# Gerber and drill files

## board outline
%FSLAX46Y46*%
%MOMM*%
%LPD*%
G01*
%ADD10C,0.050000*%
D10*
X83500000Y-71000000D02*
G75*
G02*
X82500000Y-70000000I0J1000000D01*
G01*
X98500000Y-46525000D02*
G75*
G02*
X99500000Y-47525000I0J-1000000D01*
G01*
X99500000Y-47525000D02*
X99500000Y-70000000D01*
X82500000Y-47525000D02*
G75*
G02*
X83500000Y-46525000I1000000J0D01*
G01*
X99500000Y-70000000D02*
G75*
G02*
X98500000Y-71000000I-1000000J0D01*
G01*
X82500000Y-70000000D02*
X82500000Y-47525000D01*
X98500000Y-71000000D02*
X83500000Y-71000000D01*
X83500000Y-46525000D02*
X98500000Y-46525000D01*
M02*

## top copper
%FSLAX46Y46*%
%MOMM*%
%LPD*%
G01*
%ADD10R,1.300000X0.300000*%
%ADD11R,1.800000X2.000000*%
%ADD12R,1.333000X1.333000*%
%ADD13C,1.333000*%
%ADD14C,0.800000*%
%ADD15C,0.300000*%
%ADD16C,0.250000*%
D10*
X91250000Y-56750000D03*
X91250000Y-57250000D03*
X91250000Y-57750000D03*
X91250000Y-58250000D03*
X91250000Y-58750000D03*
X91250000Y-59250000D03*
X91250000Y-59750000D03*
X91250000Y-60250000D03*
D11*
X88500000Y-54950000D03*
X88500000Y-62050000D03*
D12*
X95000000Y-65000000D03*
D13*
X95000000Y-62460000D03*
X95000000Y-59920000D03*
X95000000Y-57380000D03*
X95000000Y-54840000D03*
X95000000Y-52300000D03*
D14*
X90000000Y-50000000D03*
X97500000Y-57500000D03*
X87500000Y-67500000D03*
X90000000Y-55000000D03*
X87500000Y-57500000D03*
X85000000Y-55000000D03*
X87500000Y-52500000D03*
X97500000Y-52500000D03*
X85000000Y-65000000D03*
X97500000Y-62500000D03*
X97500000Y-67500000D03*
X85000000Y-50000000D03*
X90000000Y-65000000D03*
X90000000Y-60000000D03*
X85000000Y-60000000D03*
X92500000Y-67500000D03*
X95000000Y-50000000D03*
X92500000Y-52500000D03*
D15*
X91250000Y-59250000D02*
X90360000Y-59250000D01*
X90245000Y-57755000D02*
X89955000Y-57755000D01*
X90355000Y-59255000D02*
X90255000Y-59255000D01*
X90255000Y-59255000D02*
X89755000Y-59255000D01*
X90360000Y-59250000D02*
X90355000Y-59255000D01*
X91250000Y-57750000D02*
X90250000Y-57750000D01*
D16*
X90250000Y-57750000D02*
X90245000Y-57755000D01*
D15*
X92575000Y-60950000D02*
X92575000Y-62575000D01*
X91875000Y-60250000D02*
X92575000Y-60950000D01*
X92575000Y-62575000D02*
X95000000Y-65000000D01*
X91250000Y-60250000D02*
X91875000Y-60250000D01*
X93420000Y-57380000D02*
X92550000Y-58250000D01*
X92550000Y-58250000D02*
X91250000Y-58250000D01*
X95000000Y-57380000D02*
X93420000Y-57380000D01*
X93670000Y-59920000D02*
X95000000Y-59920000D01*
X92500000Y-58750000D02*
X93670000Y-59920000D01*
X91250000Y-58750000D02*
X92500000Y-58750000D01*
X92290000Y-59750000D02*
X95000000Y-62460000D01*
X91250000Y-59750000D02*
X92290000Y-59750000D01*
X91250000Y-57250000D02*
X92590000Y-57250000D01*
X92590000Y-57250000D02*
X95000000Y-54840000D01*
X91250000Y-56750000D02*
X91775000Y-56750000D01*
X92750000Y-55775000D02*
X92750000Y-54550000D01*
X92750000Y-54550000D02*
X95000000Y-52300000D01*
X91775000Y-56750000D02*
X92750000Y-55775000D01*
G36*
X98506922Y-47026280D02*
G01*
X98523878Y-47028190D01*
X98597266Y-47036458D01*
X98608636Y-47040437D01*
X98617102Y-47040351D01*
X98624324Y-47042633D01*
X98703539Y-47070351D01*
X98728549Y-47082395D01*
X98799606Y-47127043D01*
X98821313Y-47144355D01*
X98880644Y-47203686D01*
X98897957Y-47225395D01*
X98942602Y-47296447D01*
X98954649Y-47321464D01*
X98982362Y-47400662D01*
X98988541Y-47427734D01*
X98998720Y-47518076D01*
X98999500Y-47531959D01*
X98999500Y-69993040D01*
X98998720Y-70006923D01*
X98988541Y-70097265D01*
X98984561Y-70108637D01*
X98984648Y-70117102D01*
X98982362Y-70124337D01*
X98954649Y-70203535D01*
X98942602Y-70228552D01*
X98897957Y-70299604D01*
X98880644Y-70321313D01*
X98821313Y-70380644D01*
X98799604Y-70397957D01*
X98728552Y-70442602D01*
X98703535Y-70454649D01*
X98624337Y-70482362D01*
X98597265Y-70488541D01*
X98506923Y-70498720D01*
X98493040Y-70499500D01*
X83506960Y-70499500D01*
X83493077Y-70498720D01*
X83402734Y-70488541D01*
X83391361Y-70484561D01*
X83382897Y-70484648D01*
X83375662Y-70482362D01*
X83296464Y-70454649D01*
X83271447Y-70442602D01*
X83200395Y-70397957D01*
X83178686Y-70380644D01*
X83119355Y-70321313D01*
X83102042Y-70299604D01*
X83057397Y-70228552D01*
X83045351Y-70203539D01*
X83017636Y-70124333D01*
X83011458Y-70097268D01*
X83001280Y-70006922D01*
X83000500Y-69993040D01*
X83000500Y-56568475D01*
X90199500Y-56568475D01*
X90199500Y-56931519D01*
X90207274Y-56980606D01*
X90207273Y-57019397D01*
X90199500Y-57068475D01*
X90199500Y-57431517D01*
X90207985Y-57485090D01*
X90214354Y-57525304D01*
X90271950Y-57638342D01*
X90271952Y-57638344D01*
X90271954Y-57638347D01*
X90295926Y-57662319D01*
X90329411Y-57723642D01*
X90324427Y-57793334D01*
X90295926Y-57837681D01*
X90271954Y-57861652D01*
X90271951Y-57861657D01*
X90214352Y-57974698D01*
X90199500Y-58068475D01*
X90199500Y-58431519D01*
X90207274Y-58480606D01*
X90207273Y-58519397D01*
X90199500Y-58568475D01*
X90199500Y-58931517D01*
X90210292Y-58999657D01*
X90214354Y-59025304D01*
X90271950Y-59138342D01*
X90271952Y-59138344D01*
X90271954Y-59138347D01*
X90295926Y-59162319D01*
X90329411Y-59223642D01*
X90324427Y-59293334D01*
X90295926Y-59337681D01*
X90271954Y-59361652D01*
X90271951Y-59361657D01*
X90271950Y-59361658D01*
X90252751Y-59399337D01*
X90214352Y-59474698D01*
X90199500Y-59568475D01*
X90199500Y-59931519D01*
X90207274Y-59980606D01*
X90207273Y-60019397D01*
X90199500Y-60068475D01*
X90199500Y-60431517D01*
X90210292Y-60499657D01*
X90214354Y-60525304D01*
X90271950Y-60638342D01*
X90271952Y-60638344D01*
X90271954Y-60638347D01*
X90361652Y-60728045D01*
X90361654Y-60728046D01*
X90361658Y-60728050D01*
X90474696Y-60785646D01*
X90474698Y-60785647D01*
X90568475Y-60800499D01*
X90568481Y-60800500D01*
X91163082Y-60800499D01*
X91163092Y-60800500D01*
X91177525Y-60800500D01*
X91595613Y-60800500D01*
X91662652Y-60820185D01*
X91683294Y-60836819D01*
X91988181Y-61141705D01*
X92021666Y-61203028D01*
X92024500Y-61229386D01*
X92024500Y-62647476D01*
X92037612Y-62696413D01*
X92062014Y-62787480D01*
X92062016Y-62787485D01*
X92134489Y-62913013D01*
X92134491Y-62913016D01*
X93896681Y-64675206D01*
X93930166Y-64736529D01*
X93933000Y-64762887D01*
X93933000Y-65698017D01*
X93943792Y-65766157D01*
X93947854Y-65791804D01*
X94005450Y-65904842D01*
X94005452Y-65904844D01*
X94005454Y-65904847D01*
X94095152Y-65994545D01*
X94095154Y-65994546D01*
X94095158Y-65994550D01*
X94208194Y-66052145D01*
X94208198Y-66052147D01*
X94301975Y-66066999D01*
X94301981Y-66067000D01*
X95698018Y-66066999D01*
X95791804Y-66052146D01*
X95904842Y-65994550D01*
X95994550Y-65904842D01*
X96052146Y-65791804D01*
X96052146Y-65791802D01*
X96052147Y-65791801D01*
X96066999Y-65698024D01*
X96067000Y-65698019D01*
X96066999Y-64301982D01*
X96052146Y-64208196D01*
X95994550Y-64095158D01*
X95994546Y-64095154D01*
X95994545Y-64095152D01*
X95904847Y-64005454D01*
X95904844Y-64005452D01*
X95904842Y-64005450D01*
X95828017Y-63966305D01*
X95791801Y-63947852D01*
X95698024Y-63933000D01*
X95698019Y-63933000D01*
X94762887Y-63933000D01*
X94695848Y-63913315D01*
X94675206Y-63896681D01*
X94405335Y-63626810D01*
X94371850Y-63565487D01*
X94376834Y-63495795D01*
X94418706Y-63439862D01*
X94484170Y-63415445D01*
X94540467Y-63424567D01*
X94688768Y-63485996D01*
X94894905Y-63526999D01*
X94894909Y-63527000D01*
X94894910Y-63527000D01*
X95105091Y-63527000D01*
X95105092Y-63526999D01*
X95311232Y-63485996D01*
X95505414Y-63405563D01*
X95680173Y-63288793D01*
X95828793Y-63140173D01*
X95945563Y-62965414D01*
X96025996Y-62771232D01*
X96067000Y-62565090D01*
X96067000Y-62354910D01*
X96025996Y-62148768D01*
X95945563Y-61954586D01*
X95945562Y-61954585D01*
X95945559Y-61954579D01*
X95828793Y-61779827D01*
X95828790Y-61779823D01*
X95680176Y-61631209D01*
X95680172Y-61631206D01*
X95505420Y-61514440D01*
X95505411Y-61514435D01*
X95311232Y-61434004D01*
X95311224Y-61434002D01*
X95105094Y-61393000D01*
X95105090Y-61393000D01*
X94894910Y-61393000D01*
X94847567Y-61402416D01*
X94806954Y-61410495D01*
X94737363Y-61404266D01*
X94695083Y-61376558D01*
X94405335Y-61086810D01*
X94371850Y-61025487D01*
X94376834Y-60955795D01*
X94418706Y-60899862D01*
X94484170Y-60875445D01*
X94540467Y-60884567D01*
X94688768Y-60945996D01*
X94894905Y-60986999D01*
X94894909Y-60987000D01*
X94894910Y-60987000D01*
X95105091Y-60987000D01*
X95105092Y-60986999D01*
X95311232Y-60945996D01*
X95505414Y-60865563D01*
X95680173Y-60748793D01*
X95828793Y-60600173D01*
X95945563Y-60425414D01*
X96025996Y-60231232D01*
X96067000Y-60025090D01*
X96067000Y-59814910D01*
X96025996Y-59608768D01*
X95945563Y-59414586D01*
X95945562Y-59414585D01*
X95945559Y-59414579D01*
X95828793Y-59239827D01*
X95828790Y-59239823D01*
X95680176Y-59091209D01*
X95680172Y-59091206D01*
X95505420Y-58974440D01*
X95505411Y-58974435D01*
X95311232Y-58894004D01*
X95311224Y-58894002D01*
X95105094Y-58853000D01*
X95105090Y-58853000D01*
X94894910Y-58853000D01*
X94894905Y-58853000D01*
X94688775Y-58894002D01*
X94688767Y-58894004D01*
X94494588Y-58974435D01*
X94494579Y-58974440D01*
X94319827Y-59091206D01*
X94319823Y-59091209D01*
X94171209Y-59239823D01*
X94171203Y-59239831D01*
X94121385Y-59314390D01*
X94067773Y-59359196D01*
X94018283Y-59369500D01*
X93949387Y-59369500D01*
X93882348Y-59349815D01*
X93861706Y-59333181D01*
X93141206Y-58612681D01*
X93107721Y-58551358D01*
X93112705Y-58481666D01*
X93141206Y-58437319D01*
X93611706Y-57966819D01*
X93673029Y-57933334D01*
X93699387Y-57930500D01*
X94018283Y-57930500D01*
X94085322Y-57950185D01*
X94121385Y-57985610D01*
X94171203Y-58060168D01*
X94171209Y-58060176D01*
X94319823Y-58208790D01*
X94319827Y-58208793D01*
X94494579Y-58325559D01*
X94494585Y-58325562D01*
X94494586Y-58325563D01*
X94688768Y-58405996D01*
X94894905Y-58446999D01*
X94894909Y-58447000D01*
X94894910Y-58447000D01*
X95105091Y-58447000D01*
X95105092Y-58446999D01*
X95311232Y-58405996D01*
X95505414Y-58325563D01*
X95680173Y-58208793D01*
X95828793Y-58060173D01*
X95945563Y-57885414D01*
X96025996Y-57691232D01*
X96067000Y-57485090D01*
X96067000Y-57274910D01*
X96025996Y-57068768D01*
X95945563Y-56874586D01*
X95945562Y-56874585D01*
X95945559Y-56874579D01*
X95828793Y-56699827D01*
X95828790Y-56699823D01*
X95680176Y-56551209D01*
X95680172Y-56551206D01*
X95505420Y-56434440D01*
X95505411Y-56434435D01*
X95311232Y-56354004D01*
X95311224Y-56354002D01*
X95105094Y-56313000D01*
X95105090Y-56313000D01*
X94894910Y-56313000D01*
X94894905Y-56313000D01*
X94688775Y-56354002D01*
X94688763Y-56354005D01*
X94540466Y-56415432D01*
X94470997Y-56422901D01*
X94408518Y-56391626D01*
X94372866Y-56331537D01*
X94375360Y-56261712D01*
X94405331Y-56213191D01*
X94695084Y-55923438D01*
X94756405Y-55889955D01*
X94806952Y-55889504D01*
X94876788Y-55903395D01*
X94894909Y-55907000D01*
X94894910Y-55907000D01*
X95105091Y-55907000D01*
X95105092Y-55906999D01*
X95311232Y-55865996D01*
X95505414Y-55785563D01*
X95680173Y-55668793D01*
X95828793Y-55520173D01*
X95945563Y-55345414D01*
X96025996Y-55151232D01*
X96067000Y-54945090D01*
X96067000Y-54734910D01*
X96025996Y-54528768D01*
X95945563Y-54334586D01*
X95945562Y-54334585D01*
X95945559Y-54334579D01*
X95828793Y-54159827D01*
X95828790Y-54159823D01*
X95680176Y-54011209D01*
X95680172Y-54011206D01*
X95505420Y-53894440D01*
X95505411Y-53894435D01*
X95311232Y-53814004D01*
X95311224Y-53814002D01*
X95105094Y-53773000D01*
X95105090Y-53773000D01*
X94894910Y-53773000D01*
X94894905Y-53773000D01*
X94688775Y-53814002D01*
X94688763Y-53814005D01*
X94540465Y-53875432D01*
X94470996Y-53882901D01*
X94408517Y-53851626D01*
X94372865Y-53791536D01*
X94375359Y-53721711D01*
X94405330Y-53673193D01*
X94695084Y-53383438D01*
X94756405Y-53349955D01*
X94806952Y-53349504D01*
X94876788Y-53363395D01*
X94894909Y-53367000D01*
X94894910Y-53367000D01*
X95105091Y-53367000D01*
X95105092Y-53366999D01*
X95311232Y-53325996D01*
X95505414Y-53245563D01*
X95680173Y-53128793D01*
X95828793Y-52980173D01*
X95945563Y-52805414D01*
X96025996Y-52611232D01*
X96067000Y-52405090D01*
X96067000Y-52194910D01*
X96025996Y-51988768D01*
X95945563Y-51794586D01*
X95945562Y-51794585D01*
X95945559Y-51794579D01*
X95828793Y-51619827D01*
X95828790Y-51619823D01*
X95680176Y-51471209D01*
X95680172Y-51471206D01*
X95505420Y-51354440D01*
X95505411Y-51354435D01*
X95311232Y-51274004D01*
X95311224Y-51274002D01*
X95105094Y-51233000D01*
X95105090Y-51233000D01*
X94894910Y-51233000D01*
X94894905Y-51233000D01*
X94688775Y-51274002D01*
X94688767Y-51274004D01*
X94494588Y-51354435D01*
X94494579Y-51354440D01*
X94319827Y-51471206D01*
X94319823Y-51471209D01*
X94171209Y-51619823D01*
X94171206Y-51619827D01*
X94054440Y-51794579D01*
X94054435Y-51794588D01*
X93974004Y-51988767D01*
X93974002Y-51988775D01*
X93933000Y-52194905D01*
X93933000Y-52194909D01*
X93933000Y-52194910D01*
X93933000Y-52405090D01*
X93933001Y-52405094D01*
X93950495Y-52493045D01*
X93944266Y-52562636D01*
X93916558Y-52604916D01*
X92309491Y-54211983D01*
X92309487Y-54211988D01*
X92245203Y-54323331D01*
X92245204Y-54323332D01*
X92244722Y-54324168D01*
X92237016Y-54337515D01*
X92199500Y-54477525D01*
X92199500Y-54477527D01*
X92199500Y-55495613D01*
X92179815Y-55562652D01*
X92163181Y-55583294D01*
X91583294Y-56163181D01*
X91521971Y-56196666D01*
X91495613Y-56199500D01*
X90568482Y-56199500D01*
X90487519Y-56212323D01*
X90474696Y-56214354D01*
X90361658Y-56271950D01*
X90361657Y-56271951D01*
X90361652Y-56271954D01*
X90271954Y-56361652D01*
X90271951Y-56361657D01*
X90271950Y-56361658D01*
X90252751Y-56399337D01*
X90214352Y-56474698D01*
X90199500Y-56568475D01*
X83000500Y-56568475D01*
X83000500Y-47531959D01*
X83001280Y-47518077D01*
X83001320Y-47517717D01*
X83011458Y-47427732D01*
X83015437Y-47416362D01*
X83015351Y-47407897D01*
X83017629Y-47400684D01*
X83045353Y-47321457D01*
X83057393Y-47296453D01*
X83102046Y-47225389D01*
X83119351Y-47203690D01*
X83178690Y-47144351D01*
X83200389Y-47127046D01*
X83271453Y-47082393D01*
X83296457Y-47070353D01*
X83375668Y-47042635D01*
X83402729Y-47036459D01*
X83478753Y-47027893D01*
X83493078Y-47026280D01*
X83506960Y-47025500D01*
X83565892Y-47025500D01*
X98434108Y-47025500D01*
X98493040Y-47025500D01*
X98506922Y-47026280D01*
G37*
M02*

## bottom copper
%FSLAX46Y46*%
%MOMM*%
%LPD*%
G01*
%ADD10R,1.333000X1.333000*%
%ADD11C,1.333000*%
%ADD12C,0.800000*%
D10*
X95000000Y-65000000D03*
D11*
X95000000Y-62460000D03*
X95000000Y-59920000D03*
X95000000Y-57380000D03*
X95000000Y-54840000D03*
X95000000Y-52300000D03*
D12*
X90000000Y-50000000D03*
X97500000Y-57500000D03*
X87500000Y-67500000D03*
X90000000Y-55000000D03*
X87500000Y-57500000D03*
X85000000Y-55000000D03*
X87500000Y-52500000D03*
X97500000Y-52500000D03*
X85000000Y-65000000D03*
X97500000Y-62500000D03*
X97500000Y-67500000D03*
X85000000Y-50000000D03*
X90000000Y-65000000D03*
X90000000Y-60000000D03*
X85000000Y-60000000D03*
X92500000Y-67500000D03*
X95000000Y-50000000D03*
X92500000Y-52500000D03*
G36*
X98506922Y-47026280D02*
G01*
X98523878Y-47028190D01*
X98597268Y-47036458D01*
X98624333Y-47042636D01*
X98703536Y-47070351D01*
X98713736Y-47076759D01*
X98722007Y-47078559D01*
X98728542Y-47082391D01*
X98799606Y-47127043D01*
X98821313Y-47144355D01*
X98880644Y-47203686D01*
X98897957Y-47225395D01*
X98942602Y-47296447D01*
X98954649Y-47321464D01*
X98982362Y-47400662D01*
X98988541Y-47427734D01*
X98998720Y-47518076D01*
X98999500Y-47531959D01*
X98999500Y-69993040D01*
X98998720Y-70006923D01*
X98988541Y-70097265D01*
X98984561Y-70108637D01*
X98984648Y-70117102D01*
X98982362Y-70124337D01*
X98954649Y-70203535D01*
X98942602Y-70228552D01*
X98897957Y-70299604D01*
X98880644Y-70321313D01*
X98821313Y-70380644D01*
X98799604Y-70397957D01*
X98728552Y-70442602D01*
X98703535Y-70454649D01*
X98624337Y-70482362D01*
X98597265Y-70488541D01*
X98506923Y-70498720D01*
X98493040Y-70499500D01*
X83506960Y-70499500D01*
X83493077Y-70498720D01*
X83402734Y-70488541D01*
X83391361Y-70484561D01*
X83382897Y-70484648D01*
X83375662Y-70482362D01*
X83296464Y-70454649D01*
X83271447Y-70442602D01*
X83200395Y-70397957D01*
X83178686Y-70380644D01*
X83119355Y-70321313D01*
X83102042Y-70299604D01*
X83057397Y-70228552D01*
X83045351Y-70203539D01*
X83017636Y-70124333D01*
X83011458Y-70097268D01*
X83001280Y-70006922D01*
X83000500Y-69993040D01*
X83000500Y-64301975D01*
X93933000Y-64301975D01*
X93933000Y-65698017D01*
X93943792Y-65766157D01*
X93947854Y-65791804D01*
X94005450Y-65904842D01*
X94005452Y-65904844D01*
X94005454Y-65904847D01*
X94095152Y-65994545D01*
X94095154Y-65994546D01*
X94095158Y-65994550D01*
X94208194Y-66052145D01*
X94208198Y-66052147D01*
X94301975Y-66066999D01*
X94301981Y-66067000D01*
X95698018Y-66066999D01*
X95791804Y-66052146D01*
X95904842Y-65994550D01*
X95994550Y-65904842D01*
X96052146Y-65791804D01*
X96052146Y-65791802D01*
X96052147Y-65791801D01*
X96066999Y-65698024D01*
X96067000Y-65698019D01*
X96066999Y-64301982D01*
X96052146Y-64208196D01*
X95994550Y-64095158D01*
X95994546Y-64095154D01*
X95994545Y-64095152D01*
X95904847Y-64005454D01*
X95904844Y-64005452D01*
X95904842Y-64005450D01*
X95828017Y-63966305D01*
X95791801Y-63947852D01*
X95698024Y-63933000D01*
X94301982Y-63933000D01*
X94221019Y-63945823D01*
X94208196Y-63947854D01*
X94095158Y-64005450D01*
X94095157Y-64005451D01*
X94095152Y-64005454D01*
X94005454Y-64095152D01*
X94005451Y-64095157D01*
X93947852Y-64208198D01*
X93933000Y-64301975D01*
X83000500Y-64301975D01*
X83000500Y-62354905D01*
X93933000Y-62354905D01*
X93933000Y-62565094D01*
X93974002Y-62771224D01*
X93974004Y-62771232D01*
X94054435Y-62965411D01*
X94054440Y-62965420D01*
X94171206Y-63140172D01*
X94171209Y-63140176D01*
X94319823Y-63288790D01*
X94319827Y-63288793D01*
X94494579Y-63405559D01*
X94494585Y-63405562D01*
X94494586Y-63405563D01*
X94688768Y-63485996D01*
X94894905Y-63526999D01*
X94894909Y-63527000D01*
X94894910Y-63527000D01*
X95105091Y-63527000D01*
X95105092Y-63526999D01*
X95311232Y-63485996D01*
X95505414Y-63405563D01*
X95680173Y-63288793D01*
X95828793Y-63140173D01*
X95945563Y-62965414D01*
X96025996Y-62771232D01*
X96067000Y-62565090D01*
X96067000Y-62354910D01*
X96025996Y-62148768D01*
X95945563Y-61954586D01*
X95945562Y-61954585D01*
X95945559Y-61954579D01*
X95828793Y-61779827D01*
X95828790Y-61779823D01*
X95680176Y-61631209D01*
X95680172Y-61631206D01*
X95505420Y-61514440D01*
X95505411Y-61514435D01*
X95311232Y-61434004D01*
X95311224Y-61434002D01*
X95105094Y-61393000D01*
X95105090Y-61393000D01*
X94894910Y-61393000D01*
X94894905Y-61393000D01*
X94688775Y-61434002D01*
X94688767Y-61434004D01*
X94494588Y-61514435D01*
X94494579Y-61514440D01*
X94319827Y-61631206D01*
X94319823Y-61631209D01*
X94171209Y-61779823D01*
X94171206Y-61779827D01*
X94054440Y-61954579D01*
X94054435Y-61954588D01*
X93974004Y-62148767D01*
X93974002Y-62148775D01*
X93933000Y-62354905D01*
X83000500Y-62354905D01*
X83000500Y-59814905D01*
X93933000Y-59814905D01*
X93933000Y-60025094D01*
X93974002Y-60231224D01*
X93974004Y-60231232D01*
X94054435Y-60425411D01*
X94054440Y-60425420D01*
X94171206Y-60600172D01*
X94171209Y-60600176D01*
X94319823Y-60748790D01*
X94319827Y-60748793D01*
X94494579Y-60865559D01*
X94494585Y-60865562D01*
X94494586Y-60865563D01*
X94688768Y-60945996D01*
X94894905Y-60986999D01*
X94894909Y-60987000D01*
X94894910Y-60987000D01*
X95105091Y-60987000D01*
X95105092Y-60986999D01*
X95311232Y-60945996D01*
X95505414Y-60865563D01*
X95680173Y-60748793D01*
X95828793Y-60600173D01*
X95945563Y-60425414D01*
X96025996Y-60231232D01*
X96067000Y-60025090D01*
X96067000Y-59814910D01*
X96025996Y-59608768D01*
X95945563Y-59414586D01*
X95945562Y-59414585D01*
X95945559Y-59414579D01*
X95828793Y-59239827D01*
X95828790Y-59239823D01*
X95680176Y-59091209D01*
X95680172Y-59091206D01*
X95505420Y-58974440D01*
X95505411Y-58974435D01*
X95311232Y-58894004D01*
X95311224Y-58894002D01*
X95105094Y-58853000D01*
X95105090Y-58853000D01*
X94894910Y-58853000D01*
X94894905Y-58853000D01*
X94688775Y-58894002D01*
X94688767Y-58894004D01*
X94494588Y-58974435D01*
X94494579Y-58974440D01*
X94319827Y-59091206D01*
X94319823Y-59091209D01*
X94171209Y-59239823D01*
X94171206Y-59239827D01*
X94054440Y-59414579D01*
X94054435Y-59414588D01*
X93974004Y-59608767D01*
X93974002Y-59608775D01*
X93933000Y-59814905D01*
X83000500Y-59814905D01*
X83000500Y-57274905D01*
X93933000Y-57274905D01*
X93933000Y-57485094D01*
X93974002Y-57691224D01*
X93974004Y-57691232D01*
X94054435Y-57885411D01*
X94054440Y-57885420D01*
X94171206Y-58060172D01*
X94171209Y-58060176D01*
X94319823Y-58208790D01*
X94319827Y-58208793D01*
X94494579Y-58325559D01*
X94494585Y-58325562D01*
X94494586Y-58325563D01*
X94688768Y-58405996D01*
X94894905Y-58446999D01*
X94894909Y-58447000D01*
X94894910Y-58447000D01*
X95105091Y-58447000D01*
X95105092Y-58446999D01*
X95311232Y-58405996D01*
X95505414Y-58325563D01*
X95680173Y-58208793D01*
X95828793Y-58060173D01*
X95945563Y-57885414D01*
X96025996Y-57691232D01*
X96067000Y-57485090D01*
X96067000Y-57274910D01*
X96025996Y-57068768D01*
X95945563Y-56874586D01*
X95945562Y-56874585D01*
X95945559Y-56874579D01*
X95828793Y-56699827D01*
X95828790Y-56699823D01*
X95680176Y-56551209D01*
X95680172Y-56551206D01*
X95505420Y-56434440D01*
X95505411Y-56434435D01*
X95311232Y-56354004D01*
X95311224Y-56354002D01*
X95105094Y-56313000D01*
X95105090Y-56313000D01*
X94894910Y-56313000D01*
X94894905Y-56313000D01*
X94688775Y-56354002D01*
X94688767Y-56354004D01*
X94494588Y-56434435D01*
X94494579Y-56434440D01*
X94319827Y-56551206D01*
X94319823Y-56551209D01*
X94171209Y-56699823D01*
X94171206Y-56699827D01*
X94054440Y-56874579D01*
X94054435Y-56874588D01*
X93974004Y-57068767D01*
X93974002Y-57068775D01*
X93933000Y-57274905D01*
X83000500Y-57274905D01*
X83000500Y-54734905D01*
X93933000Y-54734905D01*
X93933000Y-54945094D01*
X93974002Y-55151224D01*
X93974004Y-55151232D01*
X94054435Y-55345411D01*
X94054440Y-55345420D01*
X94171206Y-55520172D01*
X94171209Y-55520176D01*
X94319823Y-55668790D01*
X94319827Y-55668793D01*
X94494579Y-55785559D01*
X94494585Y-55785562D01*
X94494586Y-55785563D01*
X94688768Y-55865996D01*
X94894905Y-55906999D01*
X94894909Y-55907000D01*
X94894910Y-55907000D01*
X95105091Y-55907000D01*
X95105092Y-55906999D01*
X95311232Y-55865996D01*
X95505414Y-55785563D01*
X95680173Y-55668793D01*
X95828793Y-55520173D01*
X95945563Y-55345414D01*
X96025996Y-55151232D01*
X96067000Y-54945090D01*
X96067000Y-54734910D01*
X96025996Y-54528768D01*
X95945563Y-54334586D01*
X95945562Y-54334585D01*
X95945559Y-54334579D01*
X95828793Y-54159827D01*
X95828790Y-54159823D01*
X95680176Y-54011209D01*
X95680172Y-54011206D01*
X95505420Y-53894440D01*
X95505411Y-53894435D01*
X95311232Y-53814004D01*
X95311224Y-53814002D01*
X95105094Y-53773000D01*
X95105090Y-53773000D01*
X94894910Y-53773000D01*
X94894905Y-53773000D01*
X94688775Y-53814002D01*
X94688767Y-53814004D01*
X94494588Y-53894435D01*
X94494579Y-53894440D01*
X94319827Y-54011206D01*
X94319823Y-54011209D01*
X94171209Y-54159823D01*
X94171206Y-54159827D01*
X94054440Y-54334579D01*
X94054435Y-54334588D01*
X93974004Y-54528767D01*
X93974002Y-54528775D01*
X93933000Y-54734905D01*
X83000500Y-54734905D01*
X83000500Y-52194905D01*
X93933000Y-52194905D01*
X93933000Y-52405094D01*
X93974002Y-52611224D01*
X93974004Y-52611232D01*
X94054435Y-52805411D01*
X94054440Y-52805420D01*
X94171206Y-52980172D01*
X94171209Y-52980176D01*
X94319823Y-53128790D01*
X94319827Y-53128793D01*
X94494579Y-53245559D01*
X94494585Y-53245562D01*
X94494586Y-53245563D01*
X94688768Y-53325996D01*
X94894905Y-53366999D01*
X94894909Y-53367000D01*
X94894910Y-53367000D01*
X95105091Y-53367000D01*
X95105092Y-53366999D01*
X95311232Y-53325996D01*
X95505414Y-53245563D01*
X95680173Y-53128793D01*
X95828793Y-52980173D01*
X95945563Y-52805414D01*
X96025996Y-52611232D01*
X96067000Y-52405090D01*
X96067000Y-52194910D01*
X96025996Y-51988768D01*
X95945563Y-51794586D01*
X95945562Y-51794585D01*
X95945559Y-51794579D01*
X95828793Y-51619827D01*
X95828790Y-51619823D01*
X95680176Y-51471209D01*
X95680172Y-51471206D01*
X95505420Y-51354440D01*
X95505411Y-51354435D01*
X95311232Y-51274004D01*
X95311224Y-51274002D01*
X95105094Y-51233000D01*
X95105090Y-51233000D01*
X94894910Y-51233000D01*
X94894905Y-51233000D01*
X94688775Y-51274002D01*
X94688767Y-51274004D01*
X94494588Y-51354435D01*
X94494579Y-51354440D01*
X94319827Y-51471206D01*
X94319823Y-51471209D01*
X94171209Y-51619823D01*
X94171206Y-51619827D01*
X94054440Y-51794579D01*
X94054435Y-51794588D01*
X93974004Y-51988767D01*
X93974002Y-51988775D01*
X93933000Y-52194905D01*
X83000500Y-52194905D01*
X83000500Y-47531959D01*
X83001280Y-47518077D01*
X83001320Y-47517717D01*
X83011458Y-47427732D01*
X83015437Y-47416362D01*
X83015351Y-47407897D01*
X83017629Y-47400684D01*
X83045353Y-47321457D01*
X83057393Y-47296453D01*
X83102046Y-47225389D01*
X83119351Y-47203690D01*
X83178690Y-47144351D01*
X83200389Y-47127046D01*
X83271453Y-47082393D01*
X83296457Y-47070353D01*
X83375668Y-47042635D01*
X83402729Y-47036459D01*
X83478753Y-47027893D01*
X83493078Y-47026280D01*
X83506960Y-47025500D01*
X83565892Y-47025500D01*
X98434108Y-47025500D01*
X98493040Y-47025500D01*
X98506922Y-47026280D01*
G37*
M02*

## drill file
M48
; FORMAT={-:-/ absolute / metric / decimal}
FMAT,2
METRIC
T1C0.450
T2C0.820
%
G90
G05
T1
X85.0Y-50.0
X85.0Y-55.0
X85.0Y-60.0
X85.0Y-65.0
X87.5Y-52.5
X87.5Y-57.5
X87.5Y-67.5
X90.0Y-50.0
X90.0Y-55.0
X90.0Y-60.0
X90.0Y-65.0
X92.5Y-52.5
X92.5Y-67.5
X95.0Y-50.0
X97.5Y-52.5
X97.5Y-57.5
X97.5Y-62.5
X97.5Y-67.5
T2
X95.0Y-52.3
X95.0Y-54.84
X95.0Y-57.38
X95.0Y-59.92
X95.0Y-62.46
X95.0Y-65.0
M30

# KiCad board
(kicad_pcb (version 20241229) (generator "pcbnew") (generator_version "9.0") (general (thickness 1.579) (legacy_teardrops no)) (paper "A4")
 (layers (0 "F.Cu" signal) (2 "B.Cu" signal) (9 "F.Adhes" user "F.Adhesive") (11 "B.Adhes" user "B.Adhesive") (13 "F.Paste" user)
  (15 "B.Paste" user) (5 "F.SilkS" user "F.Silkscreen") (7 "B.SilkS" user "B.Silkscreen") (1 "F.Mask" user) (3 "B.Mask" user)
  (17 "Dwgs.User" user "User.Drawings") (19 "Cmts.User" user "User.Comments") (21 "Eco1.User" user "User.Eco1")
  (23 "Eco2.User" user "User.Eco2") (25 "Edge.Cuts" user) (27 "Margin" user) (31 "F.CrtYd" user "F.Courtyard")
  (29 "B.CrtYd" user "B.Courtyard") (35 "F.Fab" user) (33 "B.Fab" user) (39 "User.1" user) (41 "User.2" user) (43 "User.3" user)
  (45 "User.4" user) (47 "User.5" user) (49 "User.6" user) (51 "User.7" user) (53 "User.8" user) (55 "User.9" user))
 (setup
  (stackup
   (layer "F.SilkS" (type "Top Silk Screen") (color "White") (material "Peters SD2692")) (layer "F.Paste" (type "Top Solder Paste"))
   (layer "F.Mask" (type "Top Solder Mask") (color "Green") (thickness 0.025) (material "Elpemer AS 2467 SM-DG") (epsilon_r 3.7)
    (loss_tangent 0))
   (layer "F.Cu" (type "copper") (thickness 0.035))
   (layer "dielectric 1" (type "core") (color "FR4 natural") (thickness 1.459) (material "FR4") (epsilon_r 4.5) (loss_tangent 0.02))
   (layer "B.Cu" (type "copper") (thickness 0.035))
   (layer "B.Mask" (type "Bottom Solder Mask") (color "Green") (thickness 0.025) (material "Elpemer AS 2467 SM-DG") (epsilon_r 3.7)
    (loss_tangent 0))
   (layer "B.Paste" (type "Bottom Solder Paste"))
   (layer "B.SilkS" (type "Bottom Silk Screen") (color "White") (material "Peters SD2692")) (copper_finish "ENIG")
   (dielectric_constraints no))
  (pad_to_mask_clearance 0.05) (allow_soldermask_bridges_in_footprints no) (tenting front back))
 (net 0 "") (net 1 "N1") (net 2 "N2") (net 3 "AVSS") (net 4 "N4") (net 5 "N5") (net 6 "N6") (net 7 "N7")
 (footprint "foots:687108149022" (layer "F.Cu") (at 88.5 58.5 -90)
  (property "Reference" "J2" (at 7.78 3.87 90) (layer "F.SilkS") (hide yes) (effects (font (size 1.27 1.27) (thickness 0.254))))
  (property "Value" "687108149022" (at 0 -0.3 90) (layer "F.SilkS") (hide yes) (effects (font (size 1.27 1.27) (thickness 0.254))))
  (pad "1" smd rect (at -1.75 -2.75 270) (size 0.3 1.3) (layers "F.Cu" "F.Mask" "F.Paste") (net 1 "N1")
   (teardrops (best_length_ratio 0.5) (max_length 1) (best_width_ratio 1) (max_width 2) (curved_edges no) (filter_ratio 0.9) (enabled yes)
    (allow_two_segments yes) (prefer_zone_connections yes)))
  (pad "2" smd rect (at -1.25 -2.75 270) (size 0.3 1.3) (layers "F.Cu" "F.Mask" "F.Paste") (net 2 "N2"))
  (pad "3" smd rect (at -0.75 -2.75 270) (size 0.3 1.3) (layers "F.Cu" "F.Mask" "F.Paste") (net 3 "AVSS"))
  (pad "4" smd rect (at -0.25 -2.75 270) (size 0.3 1.3) (layers "F.Cu" "F.Mask" "F.Paste") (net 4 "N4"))
  (pad "5" smd rect (at 0.25 -2.75 270) (size 0.3 1.3) (layers "F.Cu" "F.Mask" "F.Paste") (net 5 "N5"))
  (pad "6" smd rect (at 0.75 -2.75 270) (size 0.3 1.3) (layers "F.Cu" "F.Mask" "F.Paste") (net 3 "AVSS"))
  (pad "7" smd rect (at 1.25 -2.75 270) (size 0.3 1.3) (layers "F.Cu" "F.Mask" "F.Paste") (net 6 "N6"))
  (pad "8" smd rect (at 1.75 -2.75 270) (size 0.3 1.3) (layers "F.Cu" "F.Mask" "F.Paste") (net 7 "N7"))
  (pad "MP1" smd rect (at -3.55 0) (size 1.8 2) (layers "F.Cu" "F.Mask" "F.Paste") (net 3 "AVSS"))
  (pad "MP2" smd rect (at 3.55 0) (size 1.8 2) (layers "F.Cu" "F.Mask" "F.Paste") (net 3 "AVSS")))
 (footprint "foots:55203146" (layer "B.Cu") (at 95 65 90)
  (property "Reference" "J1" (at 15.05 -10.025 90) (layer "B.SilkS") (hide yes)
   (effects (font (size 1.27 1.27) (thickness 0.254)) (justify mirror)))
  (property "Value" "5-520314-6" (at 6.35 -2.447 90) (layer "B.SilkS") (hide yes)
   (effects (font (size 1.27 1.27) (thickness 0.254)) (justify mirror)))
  (pad "1" thru_hole rect (at 0 0 90) (size 1.333 1.333) (drill 0.82) (layers "*.Cu" "*.Mask") (remove_unused_layers no) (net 7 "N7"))
  (pad "2" thru_hole circle (at 2.54 0 90) (size 1.333 1.333) (drill 0.82) (layers "*.Cu" "*.Mask") (remove_unused_layers no) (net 6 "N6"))
  (pad "3" thru_hole circle (at 5.08 0 90) (size 1.333 1.333) (drill 0.82) (layers "*.Cu" "*.Mask") (remove_unused_layers no) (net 5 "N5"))
  (pad "4" thru_hole circle (at 7.62 0 90) (size 1.333 1.333) (drill 0.82) (layers "*.Cu" "*.Mask") (remove_unused_layers no) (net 4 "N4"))
  (pad "5" thru_hole circle (at 10.16 0 90) (size 1.333 1.333) (drill 0.82) (layers "*.Cu" "*.Mask") (remove_unused_layers no) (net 2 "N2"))
  (pad "6" thru_hole circle (at 12.7 0 90) (size 1.333 1.333) (drill 0.82) (layers "*.Cu" "*.Mask") (remove_unused_layers no) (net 1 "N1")))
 (gr_arc (start 83.5 71) (mid 82.792893 70.707107) (end 82.5 70) (stroke (width 0.05) (type default)) (layer "Edge.Cuts"))
 (gr_arc (start 98.5 46.525) (mid 99.207107 46.817893) (end 99.5 47.525) (stroke (width 0.05) (type default)) (layer "Edge.Cuts"))
 (gr_line (start 99.5 47.525) (end 99.5 70) (stroke (width 0.05) (type default)) (layer "Edge.Cuts"))
 (gr_arc (start 82.5 47.525) (mid 82.792893 46.817893) (end 83.5 46.525) (stroke (width 0.05) (type default)) (layer "Edge.Cuts"))
 (gr_arc (start 99.5 70) (mid 99.207107 70.707107) (end 98.5 71) (stroke (width 0.05) (type default)) (layer "Edge.Cuts"))
 (gr_line (start 82.5 70) (end 82.5 47.525) (stroke (width 0.05) (type default)) (layer "Edge.Cuts"))
 (gr_line (start 98.5 71) (end 83.5 71) (stroke (width 0.05) (type default)) (layer "Edge.Cuts"))
 (gr_line (start 83.5 46.525) (end 98.5 46.525) (stroke (width 0.05) (type default)) (layer "Edge.Cuts"))
 (segment (start 91.25 59.25) (end 90.36 59.25) (width 0.3) (layer "F.Cu") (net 3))
 (segment (start 90.245 57.755) (end 89.955 57.755) (width 0.3) (layer "F.Cu") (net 3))
 (segment (start 90.355 59.255) (end 90.255 59.255) (width 0.3) (layer "F.Cu") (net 3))
 (segment (start 90.255 59.255) (end 89.755 59.255) (width 0.3) (layer "F.Cu") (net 3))
 (segment (start 90.36 59.25) (end 90.355 59.255) (width 0.3) (layer "F.Cu") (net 3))
 (segment (start 91.25 57.75) (end 90.25 57.75) (width 0.3) (layer "F.Cu") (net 3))
 (segment (start 90.25 57.75) (end 90.245 57.755) (width 0.25) (layer "F.Cu") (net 3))
 (via (at 90 50) (size 0.8) (drill 0.45) (layers "F.Cu" "B.Cu") (free yes) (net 3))
 (via (at 97.5 57.5) (size 0.8) (drill 0.45) (layers "F.Cu" "B.Cu") (free yes) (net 3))
 (via (at 87.5 67.5) (size 0.8) (drill 0.45) (layers "F.Cu" "B.Cu") (free yes) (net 3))
 (via (at 90 55) (size 0.8) (drill 0.45) (layers "F.Cu" "B.Cu") (free yes) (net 3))
 (via (at 87.5 57.5) (size 0.8) (drill 0.45) (layers "F.Cu" "B.Cu") (free yes) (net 3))
 (via (at 85 55) (size 0.8) (drill 0.45) (layers "F.Cu" "B.Cu") (free yes) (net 3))
 (via (at 87.5 52.5) (size 0.8) (drill 0.45) (layers "F.Cu" "B.Cu") (free yes) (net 3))
 (via (at 97.5 52.5) (size 0.8) (drill 0.45) (layers "F.Cu" "B.Cu") (free yes) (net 3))
 (via (at 85 65) (size 0.8) (drill 0.45) (layers "F.Cu" "B.Cu") (free yes) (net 3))
 (via (at 97.5 62.5) (size 0.8) (drill 0.45) (layers "F.Cu" "B.Cu") (free yes) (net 3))
 (via (at 97.5 67.5) (size 0.8) (drill 0.45) (layers "F.Cu" "B.Cu") (free yes) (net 3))
 (via (at 85 50) (size 0.8) (drill 0.45) (layers "F.Cu" "B.Cu") (free yes) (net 3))
 (via (at 90 65) (size 0.8) (drill 0.45) (layers "F.Cu" "B.Cu") (free yes) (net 3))
 (via (at 90 60) (size 0.8) (drill 0.45) (layers "F.Cu" "B.Cu") (free yes) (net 3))
 (via (at 85 60) (size 0.8) (drill 0.45) (layers "F.Cu" "B.Cu") (free yes) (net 3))
 (via (at 92.5 67.5) (size 0.8) (drill 0.45) (layers "F.Cu" "B.Cu") (free yes) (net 3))
 (via (at 95 50) (size 0.8) (drill 0.45) (layers "F.Cu" "B.Cu") (free yes) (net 3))
 (via (at 92.5 52.5) (size 0.8) (drill 0.45) (layers "F.Cu" "B.Cu") (free yes) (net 3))
 (segment (start 92.575 60.95) (end 92.575 62.575) (width 0.3) (layer "F.Cu") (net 7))
 (segment (start 91.875 60.25) (end 92.575 60.95) (width 0.3) (layer "F.Cu") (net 7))
 (segment (start 92.575 62.575) (end 95 65) (width 0.3) (layer "F.Cu") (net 7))
 (segment (start 91.25 60.25) (end 91.875 60.25) (width 0.3) (layer "F.Cu") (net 7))
 (segment (start 93.42 57.38) (end 92.55 58.25) (width 0.3) (layer "F.Cu") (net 4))
 (segment (start 92.55 58.25) (end 91.25 58.25) (width 0.3) (layer "F.Cu") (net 4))
 (segment (start 95 57.38) (end 93.42 57.38) (width 0.3) (layer "F.Cu") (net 4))
 (segment (start 93.67 59.92) (end 95 59.92) (width 0.3) (layer "F.Cu") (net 5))
 (segment (start 92.5 58.75) (end 93.67 59.92) (width 0.3) (layer "F.Cu") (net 5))
 (segment (start 91.25 58.75) (end 92.5 58.75) (width 0.3) (layer "F.Cu") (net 5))
 (segment (start 92.29 59.75) (end 95 62.46) (width 0.3) (layer "F.Cu") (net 6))
 (segment (start 91.25 59.75) (end 92.29 59.75) (width 0.3) (layer "F.Cu") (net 6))
 (segment (start 91.25 57.25) (end 92.59 57.25) (width 0.3) (layer "F.Cu") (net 2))
 (segment (start 92.59 57.25) (end 95 54.84) (width 0.3) (layer "F.Cu") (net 2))
 (segment (start 91.25 56.75) (end 91.775 56.75) (width 0.3) (layer "F.Cu") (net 1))
 (segment (start 92.75 55.775) (end 92.75 54.55) (width 0.3) (layer "F.Cu") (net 1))
 (segment (start 92.75 54.55) (end 95 52.3) (width 0.3) (layer "F.Cu") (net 1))
 (segment (start 91.775 56.75) (end 92.75 55.775) (width 0.3) (layer "F.Cu") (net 1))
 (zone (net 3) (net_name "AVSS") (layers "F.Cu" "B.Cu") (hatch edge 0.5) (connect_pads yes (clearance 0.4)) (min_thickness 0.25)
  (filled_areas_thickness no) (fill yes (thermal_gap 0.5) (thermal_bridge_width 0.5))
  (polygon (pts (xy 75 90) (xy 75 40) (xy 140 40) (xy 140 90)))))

